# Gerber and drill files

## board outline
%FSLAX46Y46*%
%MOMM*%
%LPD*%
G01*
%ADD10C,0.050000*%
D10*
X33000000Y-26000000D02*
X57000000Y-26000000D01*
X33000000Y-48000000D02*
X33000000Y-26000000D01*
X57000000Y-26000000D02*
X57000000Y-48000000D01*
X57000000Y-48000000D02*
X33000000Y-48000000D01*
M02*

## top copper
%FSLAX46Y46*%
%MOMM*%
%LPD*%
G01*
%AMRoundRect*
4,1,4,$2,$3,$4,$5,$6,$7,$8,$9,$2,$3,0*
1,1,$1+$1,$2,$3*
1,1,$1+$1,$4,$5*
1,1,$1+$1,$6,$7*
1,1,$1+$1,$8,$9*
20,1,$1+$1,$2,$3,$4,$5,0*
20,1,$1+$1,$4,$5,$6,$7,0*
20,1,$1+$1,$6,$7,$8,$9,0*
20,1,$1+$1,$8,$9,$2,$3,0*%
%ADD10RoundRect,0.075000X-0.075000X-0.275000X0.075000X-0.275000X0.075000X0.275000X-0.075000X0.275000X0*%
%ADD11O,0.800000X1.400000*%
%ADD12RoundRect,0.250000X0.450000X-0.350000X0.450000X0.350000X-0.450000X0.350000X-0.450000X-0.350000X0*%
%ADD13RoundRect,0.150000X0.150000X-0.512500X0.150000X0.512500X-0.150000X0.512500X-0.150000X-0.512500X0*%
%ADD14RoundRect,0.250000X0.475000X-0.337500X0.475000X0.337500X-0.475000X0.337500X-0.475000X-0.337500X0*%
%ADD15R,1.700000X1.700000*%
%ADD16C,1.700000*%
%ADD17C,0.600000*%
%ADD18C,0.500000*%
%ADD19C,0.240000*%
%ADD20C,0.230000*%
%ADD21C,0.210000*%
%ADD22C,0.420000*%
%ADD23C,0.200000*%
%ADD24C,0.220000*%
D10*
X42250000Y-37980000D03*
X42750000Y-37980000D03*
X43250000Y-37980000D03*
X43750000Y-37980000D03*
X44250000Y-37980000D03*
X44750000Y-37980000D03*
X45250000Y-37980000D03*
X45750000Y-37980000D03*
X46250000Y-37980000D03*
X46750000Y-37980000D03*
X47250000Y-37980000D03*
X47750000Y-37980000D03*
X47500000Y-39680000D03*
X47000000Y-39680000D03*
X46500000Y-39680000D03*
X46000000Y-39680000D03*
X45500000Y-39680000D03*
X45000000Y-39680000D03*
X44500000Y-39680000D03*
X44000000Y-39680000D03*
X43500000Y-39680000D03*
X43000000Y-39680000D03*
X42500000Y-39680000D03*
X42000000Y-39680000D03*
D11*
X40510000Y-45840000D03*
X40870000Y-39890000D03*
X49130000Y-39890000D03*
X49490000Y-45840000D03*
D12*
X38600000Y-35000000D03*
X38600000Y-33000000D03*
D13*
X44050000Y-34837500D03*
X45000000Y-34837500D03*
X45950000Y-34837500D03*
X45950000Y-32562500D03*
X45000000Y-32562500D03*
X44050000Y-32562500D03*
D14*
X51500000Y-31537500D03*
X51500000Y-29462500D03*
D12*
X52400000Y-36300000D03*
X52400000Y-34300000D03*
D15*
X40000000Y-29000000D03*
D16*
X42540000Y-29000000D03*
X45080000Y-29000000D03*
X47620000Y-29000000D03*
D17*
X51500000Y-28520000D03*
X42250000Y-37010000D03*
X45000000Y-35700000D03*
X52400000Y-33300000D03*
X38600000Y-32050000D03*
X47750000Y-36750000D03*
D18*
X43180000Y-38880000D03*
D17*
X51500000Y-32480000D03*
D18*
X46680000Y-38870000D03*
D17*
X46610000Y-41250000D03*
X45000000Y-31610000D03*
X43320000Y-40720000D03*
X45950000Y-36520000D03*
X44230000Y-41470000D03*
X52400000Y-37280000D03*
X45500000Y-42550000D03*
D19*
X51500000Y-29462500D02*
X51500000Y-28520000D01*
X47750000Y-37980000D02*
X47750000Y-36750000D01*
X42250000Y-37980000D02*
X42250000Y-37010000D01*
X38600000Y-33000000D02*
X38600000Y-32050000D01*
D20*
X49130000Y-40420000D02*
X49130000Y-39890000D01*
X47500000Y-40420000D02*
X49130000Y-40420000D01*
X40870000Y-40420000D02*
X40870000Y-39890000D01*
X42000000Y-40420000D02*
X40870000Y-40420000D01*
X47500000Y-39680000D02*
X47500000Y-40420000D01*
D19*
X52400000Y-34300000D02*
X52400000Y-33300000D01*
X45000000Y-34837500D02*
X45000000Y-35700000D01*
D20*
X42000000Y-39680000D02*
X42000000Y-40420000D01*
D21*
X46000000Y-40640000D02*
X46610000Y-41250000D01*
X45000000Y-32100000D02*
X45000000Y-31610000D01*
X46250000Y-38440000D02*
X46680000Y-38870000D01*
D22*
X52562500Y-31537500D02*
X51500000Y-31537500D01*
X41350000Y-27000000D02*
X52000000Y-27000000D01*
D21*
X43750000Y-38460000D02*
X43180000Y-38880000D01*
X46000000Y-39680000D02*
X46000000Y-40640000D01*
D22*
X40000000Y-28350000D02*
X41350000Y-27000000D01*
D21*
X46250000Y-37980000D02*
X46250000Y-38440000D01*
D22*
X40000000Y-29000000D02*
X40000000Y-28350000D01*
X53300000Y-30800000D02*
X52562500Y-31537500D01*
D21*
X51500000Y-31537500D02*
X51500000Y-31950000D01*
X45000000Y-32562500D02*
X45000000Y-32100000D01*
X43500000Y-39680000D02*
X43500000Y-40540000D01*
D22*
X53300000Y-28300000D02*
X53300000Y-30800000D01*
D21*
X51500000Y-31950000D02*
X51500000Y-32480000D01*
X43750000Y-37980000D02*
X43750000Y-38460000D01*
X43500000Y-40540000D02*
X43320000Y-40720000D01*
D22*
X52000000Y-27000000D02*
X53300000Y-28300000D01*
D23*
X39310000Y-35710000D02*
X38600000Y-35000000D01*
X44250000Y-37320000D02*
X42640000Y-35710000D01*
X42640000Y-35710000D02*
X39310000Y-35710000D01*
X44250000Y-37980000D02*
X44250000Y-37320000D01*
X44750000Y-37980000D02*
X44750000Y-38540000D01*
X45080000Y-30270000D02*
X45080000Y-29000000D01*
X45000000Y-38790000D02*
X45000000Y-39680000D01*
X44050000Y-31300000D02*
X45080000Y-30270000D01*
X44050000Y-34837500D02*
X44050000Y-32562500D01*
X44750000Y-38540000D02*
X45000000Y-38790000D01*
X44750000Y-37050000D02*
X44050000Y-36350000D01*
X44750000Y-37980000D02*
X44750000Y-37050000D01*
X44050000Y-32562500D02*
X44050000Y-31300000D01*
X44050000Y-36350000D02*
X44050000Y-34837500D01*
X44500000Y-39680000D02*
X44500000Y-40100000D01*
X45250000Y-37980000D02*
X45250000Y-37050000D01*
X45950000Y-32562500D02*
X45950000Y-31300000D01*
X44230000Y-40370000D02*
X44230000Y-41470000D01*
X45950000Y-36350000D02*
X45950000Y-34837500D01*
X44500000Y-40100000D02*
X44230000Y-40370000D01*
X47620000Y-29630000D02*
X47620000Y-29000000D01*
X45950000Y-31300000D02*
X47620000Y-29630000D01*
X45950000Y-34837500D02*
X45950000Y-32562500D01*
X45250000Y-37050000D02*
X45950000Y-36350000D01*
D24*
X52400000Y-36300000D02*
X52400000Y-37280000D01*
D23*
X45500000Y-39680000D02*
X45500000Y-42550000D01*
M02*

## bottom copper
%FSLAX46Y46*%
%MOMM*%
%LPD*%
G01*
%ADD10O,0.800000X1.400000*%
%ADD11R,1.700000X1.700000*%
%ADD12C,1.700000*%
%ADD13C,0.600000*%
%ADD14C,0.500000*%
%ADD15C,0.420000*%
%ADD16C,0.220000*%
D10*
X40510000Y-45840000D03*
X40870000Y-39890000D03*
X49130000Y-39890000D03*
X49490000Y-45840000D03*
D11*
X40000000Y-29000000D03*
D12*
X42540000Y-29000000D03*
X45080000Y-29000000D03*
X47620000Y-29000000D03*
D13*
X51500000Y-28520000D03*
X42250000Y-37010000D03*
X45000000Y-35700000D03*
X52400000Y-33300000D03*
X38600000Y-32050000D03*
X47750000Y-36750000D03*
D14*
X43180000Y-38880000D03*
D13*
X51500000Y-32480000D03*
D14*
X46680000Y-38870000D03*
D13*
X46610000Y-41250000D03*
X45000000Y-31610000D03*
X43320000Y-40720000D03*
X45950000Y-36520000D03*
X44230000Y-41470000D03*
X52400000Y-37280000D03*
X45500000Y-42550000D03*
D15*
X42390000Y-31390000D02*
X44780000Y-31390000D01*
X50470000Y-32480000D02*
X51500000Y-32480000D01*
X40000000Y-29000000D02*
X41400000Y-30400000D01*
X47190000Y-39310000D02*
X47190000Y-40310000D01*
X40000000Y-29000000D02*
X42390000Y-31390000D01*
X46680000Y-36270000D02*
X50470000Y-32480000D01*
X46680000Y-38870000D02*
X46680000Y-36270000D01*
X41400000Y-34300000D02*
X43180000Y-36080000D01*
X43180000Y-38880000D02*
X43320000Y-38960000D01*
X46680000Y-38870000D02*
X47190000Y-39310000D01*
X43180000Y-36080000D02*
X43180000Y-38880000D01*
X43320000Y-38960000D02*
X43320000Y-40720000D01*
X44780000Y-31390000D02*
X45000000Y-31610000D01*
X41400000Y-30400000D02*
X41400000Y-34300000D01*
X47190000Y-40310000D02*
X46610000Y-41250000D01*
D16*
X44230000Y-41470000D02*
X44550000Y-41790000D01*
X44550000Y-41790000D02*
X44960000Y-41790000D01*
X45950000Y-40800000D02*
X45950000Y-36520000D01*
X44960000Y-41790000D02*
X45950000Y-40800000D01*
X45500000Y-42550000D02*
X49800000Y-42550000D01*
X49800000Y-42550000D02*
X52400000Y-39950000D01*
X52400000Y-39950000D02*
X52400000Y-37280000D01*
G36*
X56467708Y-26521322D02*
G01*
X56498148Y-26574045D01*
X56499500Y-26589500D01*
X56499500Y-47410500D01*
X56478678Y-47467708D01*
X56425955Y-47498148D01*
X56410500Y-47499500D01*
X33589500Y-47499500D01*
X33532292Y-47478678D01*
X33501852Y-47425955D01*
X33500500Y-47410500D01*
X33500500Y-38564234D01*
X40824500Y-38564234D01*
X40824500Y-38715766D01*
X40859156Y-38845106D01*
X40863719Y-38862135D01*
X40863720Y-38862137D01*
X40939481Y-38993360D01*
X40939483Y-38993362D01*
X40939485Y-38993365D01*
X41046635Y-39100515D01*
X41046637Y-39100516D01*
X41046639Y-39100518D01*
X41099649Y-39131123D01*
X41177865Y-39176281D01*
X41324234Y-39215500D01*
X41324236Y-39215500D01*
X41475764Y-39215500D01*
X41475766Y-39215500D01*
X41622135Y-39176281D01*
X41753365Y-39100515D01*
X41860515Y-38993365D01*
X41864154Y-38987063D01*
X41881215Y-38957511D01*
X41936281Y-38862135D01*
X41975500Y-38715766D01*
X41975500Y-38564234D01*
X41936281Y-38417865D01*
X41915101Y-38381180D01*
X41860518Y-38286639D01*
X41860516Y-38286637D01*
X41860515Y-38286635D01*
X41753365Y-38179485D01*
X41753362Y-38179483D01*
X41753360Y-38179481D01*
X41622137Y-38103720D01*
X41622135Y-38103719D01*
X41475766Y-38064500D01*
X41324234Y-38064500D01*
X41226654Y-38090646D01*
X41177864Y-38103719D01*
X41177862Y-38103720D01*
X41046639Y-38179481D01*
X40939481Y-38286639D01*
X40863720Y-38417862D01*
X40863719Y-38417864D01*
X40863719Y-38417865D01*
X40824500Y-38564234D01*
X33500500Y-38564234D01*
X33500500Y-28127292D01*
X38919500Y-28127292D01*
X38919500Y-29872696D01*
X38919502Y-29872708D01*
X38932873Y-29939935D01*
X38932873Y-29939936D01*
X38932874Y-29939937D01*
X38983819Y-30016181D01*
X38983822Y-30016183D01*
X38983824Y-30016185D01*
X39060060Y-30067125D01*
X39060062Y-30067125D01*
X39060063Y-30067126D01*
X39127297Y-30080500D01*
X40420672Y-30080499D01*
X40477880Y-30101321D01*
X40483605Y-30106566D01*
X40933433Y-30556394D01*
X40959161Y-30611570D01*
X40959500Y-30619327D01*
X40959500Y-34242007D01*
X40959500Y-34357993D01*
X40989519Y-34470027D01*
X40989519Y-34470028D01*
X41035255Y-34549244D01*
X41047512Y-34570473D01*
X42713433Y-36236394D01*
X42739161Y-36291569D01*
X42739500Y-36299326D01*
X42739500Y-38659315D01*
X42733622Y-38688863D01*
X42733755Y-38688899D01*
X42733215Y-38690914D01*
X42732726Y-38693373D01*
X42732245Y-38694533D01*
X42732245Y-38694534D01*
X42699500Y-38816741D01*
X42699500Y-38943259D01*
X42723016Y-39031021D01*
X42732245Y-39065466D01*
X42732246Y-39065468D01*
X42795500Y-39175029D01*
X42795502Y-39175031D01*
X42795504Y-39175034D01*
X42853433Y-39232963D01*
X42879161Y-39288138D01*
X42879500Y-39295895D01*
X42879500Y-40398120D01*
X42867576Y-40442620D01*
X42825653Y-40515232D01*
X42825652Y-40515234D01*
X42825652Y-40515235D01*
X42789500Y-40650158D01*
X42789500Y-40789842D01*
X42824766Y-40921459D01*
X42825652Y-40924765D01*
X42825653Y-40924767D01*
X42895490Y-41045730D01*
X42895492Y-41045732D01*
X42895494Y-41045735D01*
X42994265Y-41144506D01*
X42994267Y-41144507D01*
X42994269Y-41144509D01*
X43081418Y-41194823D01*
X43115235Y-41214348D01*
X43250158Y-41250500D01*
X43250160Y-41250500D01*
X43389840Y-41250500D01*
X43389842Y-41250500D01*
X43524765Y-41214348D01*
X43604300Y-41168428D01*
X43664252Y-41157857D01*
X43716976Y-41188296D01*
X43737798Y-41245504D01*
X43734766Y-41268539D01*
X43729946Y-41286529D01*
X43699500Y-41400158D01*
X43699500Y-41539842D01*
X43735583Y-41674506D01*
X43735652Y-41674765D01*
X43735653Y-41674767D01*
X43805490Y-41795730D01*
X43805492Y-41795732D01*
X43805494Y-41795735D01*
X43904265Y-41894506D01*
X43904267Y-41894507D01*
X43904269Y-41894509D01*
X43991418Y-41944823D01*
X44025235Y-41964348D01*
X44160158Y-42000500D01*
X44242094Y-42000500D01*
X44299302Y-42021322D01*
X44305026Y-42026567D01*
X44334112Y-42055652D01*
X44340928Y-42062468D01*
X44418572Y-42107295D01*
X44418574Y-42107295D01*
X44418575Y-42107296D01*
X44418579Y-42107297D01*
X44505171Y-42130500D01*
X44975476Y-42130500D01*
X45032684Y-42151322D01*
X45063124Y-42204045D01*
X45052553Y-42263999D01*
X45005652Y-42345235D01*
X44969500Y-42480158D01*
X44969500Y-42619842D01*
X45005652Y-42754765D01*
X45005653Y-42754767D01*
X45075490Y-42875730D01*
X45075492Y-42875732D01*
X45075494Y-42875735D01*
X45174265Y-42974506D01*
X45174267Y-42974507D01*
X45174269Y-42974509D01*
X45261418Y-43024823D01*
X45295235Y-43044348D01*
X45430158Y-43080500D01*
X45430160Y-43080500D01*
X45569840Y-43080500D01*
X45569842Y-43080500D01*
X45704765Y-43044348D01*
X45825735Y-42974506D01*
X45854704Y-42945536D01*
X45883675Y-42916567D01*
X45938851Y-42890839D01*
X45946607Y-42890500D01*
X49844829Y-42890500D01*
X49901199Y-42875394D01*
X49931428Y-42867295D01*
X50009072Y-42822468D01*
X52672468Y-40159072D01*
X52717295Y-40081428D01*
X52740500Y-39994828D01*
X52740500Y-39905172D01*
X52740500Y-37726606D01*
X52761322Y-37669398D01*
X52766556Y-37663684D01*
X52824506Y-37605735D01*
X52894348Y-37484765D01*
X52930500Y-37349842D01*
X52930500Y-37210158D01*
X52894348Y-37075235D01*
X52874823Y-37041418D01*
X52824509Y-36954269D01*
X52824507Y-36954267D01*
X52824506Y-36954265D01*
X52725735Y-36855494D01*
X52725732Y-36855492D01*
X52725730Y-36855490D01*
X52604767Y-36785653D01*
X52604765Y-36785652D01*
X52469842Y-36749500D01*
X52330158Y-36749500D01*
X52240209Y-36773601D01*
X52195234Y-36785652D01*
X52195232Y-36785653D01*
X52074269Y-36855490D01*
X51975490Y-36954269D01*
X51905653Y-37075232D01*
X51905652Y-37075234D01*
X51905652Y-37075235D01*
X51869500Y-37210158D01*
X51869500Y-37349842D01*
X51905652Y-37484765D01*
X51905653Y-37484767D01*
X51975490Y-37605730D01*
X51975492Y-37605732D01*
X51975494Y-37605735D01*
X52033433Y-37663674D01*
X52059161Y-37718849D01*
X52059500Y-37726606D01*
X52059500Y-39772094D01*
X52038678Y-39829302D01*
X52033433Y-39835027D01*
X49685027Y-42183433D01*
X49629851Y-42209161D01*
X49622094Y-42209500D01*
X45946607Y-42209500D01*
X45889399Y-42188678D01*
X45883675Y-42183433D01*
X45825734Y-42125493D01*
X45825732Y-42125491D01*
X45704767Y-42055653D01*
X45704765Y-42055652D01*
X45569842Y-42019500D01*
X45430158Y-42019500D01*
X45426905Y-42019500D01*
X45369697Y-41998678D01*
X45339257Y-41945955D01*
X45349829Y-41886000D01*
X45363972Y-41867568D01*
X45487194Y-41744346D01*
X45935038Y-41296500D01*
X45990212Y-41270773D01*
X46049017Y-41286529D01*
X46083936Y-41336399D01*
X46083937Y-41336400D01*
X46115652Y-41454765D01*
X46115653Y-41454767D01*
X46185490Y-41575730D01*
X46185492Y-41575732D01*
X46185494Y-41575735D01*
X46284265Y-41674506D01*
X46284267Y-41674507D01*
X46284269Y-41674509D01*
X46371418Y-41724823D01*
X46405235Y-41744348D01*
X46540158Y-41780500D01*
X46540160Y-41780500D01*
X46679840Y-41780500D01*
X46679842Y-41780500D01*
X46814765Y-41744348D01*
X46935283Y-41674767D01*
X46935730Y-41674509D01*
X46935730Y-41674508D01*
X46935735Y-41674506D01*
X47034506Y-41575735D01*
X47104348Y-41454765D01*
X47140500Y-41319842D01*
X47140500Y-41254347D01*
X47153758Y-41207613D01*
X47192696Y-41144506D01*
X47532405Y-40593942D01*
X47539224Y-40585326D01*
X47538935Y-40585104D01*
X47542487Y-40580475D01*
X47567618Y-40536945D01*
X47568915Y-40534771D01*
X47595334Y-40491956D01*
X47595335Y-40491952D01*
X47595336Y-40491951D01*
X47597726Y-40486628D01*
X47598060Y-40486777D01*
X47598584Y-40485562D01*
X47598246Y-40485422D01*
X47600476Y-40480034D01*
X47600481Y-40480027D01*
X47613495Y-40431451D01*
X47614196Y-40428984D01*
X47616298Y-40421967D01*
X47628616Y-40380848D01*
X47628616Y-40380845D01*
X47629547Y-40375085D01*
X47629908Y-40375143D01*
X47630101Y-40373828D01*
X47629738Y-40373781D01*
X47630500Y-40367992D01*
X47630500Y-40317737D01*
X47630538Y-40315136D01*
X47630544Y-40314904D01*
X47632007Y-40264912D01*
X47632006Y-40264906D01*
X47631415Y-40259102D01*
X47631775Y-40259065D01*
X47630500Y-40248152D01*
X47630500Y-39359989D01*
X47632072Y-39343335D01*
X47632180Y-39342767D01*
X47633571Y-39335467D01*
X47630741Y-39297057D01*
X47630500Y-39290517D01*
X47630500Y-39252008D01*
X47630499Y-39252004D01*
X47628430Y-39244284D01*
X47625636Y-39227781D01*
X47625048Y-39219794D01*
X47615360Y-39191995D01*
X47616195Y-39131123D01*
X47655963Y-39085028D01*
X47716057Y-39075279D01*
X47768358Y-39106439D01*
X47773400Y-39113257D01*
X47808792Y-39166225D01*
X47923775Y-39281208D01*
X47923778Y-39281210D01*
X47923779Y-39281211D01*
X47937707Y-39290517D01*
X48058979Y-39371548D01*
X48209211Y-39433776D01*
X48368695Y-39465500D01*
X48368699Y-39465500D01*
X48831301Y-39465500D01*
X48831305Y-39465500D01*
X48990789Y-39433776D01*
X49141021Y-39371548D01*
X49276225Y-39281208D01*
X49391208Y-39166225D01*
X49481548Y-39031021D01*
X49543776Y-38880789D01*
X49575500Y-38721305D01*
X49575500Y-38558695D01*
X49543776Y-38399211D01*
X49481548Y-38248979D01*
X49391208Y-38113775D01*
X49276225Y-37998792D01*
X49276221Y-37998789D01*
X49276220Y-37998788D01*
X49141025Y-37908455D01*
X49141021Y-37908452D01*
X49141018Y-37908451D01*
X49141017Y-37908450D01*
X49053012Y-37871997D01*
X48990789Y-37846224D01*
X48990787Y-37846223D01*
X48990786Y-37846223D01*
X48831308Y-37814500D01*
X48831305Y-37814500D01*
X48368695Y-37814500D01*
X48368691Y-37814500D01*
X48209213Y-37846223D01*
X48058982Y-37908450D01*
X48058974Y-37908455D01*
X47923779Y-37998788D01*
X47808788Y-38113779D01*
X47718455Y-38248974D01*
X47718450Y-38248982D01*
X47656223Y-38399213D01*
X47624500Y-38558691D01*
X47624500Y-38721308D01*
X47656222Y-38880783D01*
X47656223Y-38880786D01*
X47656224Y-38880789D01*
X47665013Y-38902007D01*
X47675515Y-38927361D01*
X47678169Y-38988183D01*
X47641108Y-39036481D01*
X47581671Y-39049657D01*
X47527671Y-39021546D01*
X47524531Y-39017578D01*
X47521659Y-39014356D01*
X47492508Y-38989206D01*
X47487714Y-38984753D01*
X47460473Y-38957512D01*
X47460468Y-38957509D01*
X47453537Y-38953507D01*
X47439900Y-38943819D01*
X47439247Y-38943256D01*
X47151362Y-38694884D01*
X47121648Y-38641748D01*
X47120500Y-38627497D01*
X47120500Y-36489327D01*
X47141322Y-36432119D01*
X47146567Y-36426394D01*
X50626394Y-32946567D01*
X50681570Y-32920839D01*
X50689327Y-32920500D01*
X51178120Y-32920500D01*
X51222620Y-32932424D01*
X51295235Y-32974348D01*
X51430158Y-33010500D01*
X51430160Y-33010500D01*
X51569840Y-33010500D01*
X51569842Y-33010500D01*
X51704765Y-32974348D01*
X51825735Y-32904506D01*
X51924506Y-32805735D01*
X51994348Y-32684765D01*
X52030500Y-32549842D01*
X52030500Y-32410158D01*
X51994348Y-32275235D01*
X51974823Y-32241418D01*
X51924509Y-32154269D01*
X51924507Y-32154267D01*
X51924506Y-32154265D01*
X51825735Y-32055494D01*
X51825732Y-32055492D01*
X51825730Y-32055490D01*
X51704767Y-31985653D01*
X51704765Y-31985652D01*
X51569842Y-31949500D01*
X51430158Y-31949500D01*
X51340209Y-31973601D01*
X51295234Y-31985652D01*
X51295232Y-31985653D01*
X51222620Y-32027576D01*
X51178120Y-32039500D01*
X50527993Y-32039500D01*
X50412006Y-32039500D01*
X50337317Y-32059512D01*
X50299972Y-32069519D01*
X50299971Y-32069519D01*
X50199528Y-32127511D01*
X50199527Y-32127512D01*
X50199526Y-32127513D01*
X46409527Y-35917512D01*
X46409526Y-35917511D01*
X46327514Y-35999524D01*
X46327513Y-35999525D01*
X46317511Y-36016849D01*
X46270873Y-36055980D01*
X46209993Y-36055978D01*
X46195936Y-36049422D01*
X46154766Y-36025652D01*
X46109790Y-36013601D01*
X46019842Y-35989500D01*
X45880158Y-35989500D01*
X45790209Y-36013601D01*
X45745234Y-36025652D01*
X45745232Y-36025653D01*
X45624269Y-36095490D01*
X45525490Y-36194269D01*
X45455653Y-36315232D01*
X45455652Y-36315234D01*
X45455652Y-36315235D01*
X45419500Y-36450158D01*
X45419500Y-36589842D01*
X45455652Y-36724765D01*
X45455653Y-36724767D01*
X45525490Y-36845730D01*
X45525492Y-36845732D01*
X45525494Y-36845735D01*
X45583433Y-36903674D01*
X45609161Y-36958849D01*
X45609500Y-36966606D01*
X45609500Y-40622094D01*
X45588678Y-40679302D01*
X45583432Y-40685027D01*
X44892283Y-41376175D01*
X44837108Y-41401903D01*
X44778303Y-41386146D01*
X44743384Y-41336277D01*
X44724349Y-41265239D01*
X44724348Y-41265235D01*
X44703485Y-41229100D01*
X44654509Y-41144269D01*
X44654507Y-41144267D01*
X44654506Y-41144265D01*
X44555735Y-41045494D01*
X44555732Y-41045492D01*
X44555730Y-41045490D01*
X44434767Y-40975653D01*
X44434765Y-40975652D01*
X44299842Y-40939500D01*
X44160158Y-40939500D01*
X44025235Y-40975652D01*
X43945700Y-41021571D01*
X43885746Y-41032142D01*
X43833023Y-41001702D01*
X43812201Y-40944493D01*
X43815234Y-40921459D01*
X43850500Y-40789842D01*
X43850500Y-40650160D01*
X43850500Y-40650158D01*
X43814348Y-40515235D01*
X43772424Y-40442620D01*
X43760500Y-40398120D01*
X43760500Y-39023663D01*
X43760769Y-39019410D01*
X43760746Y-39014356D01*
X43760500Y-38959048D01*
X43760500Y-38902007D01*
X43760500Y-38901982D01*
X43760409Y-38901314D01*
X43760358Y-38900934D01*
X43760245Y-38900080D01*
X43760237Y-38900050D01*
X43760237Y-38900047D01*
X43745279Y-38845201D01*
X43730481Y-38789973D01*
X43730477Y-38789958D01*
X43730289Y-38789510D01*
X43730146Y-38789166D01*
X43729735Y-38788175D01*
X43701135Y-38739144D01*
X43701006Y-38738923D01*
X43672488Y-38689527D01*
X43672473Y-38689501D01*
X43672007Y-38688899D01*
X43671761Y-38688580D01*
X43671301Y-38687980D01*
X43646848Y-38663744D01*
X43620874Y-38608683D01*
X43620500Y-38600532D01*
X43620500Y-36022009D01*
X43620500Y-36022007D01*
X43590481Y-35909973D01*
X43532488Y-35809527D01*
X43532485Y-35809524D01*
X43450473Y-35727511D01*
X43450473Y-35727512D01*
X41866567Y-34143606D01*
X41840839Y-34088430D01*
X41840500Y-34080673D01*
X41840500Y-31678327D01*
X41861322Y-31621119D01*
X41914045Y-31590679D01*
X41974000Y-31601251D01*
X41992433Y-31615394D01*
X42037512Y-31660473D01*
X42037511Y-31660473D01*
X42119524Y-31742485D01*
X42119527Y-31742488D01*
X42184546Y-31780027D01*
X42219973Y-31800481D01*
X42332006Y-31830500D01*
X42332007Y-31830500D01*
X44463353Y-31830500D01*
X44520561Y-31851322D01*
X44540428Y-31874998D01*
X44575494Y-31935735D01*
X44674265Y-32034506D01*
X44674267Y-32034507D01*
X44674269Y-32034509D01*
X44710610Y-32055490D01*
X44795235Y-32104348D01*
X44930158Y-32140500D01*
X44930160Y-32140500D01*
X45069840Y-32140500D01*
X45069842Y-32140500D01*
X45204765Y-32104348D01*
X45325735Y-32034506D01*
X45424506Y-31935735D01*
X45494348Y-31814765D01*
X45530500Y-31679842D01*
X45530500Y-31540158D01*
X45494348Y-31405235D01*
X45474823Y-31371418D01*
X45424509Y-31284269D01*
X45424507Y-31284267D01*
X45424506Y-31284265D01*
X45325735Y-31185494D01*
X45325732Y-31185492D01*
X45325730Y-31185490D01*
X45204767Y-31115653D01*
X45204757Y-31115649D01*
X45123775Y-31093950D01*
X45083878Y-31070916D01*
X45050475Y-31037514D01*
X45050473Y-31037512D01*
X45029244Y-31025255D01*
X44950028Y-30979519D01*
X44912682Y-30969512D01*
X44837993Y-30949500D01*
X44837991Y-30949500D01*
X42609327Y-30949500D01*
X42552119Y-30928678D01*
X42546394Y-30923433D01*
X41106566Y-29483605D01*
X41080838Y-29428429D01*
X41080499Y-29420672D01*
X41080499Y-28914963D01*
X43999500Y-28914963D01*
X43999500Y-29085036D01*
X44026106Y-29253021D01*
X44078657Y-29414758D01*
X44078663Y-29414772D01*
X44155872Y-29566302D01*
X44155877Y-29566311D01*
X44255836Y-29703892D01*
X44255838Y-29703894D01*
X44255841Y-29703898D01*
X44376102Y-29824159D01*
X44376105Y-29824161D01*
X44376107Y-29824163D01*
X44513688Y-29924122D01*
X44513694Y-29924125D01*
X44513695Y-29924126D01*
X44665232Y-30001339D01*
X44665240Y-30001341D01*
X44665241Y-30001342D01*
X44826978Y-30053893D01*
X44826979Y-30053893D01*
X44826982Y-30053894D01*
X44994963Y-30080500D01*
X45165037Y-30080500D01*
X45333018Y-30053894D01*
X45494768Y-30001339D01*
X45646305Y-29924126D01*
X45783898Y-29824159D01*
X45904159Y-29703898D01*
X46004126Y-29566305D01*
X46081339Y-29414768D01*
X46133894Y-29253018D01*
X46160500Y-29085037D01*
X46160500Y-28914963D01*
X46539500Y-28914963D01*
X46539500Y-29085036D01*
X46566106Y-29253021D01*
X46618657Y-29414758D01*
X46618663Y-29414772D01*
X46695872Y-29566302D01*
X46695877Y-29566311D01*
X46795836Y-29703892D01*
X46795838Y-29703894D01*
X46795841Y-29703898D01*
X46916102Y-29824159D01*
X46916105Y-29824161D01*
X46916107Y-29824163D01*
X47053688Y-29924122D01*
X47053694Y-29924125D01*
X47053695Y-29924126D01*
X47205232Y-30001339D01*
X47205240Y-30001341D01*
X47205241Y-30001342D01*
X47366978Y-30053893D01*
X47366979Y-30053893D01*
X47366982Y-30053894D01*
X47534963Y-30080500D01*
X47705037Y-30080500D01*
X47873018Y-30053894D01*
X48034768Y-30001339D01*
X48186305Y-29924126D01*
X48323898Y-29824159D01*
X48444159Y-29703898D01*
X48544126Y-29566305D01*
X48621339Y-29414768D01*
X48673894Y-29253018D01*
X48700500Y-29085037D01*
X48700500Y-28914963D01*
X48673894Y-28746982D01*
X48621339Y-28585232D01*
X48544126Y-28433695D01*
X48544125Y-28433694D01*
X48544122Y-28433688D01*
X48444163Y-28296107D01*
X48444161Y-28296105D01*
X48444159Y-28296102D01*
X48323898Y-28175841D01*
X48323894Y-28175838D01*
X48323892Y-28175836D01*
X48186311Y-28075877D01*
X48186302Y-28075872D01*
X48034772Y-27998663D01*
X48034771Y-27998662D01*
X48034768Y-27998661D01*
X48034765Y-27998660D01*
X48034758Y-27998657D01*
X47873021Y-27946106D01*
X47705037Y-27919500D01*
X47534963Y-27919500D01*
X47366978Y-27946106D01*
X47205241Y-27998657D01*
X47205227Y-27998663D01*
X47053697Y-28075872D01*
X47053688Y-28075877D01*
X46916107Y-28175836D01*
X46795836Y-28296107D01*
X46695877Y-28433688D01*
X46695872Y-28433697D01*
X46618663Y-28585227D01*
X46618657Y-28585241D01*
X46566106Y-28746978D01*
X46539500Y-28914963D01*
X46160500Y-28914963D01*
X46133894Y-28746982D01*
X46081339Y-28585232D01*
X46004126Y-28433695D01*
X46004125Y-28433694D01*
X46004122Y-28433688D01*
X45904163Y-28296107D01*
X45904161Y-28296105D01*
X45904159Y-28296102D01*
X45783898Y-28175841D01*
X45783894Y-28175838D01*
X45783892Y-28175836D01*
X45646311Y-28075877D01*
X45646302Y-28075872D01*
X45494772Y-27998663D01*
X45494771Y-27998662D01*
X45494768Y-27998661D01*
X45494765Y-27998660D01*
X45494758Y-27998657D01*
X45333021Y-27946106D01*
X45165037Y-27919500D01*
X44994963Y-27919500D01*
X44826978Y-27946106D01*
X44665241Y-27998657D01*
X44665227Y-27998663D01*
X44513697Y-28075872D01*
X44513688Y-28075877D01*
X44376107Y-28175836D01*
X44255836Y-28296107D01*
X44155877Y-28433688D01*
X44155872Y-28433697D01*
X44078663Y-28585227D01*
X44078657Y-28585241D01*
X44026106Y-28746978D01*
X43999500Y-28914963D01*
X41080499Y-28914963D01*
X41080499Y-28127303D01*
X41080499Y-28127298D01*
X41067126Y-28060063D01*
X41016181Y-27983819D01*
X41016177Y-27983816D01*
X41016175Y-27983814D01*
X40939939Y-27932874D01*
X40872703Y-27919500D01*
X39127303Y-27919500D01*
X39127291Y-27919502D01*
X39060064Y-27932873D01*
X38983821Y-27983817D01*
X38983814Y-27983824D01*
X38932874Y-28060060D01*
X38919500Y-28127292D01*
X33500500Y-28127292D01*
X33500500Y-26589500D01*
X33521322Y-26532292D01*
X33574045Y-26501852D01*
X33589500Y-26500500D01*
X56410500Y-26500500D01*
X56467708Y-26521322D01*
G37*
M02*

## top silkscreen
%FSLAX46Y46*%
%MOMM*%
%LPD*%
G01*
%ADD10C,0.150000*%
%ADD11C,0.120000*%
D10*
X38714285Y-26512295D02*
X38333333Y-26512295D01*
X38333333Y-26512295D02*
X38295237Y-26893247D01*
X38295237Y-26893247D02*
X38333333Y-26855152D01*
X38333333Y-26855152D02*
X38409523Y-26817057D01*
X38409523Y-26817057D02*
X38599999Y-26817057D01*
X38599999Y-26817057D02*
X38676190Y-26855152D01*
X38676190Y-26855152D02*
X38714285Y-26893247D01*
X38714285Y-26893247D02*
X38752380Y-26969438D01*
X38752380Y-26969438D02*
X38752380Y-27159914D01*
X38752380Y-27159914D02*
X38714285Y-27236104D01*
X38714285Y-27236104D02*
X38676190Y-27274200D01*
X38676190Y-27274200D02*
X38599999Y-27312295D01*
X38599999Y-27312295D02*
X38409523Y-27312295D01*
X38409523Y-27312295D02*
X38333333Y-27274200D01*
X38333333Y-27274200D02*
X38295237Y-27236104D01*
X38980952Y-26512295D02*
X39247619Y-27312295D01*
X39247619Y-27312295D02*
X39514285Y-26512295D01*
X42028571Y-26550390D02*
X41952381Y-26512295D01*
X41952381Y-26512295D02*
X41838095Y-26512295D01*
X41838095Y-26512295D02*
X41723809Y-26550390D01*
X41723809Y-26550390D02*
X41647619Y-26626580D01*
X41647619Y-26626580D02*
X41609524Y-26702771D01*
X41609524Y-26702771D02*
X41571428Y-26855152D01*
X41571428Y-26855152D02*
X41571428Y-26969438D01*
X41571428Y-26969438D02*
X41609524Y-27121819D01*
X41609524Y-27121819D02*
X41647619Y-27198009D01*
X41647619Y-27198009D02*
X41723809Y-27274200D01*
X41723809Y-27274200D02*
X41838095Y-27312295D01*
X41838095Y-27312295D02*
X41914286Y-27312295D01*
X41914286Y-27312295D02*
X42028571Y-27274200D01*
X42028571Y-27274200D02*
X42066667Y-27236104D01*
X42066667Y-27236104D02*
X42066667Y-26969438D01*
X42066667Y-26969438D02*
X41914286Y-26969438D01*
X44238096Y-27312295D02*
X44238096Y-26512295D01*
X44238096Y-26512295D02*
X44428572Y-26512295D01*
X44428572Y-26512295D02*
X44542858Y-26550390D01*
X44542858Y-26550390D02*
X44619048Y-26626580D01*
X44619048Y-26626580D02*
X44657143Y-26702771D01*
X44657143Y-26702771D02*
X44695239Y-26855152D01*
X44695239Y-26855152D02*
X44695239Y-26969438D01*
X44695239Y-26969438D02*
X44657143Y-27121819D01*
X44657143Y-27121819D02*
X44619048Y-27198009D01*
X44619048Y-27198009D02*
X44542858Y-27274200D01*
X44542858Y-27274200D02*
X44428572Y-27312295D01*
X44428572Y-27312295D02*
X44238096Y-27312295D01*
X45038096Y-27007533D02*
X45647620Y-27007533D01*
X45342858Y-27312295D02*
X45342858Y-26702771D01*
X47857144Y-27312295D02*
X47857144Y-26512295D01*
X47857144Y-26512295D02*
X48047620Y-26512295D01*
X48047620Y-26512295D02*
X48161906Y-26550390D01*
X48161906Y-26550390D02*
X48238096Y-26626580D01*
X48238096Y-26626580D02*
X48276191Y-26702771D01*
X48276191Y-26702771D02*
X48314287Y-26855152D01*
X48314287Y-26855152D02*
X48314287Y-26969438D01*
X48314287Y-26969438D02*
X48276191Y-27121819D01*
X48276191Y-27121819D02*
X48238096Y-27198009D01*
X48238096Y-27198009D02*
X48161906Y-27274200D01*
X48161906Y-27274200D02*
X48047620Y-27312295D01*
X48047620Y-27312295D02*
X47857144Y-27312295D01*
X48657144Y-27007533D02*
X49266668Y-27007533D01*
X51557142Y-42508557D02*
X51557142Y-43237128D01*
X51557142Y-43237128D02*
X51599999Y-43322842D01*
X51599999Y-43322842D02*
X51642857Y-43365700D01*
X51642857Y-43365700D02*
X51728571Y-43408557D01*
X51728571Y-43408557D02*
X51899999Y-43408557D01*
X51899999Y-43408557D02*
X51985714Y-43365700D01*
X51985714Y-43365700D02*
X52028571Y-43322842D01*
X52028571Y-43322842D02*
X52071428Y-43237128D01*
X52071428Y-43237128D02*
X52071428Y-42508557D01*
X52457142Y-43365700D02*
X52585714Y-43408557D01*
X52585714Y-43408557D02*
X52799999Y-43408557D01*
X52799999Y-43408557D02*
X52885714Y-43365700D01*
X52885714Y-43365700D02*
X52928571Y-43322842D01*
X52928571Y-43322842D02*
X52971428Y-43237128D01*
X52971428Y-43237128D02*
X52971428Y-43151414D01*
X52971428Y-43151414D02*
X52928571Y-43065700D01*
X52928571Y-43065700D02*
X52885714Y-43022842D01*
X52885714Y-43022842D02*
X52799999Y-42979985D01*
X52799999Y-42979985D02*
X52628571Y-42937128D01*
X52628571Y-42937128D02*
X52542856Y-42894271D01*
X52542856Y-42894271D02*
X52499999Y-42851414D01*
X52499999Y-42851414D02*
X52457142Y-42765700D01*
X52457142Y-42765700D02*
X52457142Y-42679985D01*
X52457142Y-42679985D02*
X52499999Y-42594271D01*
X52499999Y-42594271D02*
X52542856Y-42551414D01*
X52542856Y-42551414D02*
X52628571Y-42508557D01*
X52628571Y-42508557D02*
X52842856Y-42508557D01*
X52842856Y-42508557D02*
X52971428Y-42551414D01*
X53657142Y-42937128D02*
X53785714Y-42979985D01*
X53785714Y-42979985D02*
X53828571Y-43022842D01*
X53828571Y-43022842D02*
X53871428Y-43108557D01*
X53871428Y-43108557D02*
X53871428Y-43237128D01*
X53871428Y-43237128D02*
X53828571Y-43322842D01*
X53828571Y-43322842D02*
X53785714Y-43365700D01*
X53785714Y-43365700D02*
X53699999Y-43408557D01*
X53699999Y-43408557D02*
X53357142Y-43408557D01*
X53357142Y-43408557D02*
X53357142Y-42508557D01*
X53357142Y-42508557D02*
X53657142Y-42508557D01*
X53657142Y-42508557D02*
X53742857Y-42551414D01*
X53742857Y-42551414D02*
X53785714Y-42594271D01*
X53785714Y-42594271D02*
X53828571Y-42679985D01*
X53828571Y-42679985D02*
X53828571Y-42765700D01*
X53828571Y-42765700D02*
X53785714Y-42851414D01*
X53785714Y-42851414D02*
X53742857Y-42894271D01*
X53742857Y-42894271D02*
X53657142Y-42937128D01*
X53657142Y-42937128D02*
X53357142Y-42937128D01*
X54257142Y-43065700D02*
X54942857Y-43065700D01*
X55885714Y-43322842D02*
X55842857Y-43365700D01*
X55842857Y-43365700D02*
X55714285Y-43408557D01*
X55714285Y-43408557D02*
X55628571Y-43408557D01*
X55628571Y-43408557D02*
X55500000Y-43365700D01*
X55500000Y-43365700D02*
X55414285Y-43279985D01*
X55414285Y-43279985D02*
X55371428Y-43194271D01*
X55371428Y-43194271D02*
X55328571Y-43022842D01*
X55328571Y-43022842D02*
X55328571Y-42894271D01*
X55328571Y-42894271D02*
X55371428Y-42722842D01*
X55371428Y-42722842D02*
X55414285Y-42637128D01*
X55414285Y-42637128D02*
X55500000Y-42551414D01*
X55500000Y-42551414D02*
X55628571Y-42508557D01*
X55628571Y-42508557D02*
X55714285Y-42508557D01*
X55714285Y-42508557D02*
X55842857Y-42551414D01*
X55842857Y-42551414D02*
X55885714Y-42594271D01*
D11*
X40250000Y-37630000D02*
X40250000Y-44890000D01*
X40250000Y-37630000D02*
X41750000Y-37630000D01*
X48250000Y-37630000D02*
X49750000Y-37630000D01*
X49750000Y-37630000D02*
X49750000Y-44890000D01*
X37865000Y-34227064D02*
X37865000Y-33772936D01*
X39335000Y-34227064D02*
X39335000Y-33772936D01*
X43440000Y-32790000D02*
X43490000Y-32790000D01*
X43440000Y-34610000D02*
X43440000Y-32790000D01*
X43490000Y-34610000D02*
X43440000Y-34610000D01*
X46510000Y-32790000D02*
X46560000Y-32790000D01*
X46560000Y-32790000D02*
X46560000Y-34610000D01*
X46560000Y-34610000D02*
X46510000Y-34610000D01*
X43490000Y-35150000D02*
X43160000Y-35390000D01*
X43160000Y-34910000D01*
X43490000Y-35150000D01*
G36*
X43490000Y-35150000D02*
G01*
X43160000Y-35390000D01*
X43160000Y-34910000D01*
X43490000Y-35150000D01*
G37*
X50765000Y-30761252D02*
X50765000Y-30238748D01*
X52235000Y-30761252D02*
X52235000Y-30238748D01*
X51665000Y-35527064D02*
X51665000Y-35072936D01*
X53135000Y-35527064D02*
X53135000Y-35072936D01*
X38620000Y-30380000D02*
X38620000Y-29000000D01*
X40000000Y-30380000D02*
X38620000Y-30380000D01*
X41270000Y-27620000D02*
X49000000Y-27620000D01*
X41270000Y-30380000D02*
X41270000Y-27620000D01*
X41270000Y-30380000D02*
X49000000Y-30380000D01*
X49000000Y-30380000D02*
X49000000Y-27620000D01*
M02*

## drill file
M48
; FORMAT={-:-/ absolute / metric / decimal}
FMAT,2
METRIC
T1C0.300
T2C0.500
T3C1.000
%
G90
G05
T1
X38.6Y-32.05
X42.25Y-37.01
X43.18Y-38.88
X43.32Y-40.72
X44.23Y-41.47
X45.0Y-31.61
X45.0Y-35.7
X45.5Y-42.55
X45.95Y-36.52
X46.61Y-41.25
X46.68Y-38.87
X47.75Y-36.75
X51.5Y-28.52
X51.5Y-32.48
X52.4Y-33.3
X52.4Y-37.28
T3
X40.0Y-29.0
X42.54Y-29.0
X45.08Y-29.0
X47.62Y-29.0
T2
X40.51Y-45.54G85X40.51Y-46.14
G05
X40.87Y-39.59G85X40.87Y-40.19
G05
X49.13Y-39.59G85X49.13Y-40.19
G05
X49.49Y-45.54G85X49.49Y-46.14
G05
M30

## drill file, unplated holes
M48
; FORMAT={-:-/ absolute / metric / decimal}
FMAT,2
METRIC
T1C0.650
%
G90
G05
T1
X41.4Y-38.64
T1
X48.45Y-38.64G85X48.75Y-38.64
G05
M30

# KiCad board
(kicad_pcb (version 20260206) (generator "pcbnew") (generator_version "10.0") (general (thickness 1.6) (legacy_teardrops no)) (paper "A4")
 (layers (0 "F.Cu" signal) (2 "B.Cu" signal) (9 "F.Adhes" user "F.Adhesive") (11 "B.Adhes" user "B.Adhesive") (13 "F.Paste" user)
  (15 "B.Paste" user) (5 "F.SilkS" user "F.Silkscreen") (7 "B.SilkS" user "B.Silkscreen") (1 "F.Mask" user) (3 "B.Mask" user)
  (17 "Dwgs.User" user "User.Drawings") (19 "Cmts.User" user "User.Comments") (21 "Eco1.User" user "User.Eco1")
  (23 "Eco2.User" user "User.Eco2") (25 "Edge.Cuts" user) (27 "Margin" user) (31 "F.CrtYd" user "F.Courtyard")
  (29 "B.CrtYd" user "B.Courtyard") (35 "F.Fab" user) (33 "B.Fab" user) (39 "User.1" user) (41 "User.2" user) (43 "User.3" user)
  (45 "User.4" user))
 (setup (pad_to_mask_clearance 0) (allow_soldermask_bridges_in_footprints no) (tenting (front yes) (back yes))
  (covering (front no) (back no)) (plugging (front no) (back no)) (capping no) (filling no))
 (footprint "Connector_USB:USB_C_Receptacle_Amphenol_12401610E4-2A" (layer "F.Cu") (at 45 43)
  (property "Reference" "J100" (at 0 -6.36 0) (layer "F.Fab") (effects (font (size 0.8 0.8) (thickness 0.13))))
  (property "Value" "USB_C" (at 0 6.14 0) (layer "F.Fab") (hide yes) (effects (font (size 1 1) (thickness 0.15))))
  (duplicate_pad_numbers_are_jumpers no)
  (fp_line (start -4.75 -5.37) (end -4.75 1.89) (stroke (width 0.12) (type solid)) (layer "F.SilkS"))
  (fp_line (start -4.75 -5.37) (end -3.25 -5.37) (stroke (width 0.12) (type solid)) (layer "F.SilkS"))
  (fp_line (start 3.25 -5.37) (end 4.75 -5.37) (stroke (width 0.12) (type solid)) (layer "F.SilkS"))
  (fp_line (start 4.75 -5.37) (end 4.75 1.89) (stroke (width 0.12) (type solid)) (layer "F.SilkS"))
  (pad "" np_thru_hole circle (at -3.6 -4.36) (size 0.65 0.65) (drill 0.65) (layers "*.Cu" "*.Mask"))
  (pad "" np_thru_hole oval (at 3.6 -4.36) (size 0.95 0.65) (drill oval 0.95 0.65) (layers "*.Cu" "*.Mask"))
  (pad "A1" smd roundrect (at -2.75 -5.02) (size 0.3 0.7) (layers "F.Cu" "F.Mask" "F.Paste") (roundrect_rratio 0.25) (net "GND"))
  (pad "A2" smd roundrect (at -2.25 -5.02) (size 0.3 0.7) (layers "F.Cu" "F.Mask" "F.Paste") (roundrect_rratio 0.25))
  (pad "A3" smd roundrect (at -1.75 -5.02) (size 0.3 0.7) (layers "F.Cu" "F.Mask" "F.Paste") (roundrect_rratio 0.25))
  (pad "A4" smd roundrect (at -1.25 -5.02) (size 0.3 0.7) (layers "F.Cu" "F.Mask" "F.Paste") (roundrect_rratio 0.25) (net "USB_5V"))
  (pad "A5" smd roundrect (at -0.75 -5.02) (size 0.3 0.7) (layers "F.Cu" "F.Mask" "F.Paste") (roundrect_rratio 0.25) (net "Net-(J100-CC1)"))
  (pad "A6" smd roundrect (at -0.25 -5.02) (size 0.3 0.7) (layers "F.Cu" "F.Mask" "F.Paste") (roundrect_rratio 0.25) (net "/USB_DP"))
  (pad "A7" smd roundrect (at 0.25 -5.02) (size 0.3 0.7) (layers "F.Cu" "F.Mask" "F.Paste") (roundrect_rratio 0.25) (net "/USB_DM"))
  (pad "A8" smd roundrect (at 0.75 -5.02) (size 0.3 0.7) (layers "F.Cu" "F.Mask" "F.Paste") (roundrect_rratio 0.25))
  (pad "A9" smd roundrect (at 1.25 -5.02) (size 0.3 0.7) (layers "F.Cu" "F.Mask" "F.Paste") (roundrect_rratio 0.25) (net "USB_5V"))
  (pad "A10" smd roundrect (at 1.75 -5.02) (size 0.3 0.7) (layers "F.Cu" "F.Mask" "F.Paste") (roundrect_rratio 0.25))
  (pad "A11" smd roundrect (at 2.25 -5.02) (size 0.3 0.7) (layers "F.Cu" "F.Mask" "F.Paste") (roundrect_rratio 0.25))
  (pad "A12" smd roundrect (at 2.75 -5.02) (size 0.3 0.7) (layers "F.Cu" "F.Mask" "F.Paste") (roundrect_rratio 0.25) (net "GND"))
  (pad "B1" smd roundrect (at 2.5 -3.32) (size 0.3 0.7) (layers "F.Cu" "F.Mask" "F.Paste") (roundrect_rratio 0.25) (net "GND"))
  (pad "B2" smd roundrect (at 2 -3.32) (size 0.3 0.7) (layers "F.Cu" "F.Mask" "F.Paste") (roundrect_rratio 0.25))
  (pad "B3" smd roundrect (at 1.5 -3.32) (size 0.3 0.7) (layers "F.Cu" "F.Mask" "F.Paste") (roundrect_rratio 0.25))
  (pad "B4" smd roundrect (at 1 -3.32) (size 0.3 0.7) (layers "F.Cu" "F.Mask" "F.Paste") (roundrect_rratio 0.25) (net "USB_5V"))
  (pad "B5" smd roundrect (at 0.5 -3.32) (size 0.3 0.7) (layers "F.Cu" "F.Mask" "F.Paste") (roundrect_rratio 0.25) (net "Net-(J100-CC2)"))
  (pad "B6" smd roundrect (at 0 -3.32) (size 0.3 0.7) (layers "F.Cu" "F.Mask" "F.Paste") (roundrect_rratio 0.25) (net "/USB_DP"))
  (pad "B7" smd roundrect (at -0.5 -3.32) (size 0.3 0.7) (layers "F.Cu" "F.Mask" "F.Paste") (roundrect_rratio 0.25) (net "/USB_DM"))
  (pad "B8" smd roundrect (at -1 -3.32) (size 0.3 0.7) (layers "F.Cu" "F.Mask" "F.Paste") (roundrect_rratio 0.25))
  (pad "B9" smd roundrect (at -1.5 -3.32) (size 0.3 0.7) (layers "F.Cu" "F.Mask" "F.Paste") (roundrect_rratio 0.25) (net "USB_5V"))
  (pad "B10" smd roundrect (at -2 -3.32) (size 0.3 0.7) (layers "F.Cu" "F.Mask" "F.Paste") (roundrect_rratio 0.25))
  (pad "B11" smd roundrect (at -2.5 -3.32) (size 0.3 0.7) (layers "F.Cu" "F.Mask" "F.Paste") (roundrect_rratio 0.25))
  (pad "B12" smd roundrect (at -3 -3.32) (size 0.3 0.7) (layers "F.Cu" "F.Mask" "F.Paste") (roundrect_rratio 0.25) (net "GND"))
  (pad "SH" thru_hole oval (at -4.49 2.84) (size 0.8 1.4) (drill oval 0.5 1.1) (layers "*.Cu" "*.Mask") (remove_unused_layers no)
   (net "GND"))
  (pad "SH" thru_hole oval (at -4.13 -3.11) (size 0.8 1.4) (drill oval 0.5 1.1) (layers "*.Cu" "*.Mask") (remove_unused_layers no)
   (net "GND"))
  (pad "SH" thru_hole oval (at 4.13 -3.11) (size 0.8 1.4) (drill oval 0.5 1.1) (layers "*.Cu" "*.Mask") (remove_unused_layers no)
   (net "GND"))
  (pad "SH" thru_hole oval (at 4.49 2.84) (size 0.8 1.4) (drill oval 0.5 1.1) (layers "*.Cu" "*.Mask") (remove_unused_layers no) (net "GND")))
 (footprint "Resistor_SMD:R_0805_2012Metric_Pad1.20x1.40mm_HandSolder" (layer "F.Cu") (at 38.6 34 90)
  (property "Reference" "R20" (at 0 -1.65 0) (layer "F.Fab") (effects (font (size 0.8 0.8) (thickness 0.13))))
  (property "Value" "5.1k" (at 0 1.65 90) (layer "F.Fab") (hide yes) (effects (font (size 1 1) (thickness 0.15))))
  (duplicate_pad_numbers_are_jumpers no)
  (fp_line (start -0.227064 -0.735) (end 0.227064 -0.735) (stroke (width 0.12) (type solid)) (layer "F.SilkS"))
  (fp_line (start -0.227064 0.735) (end 0.227064 0.735) (stroke (width 0.12) (type solid)) (layer "F.SilkS"))
  (pad "1" smd roundrect (at -1 0 90) (size 1.2 1.4) (layers "F.Cu" "F.Mask" "F.Paste") (roundrect_rratio 0.208333) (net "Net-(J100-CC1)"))
  (pad "2" smd roundrect (at 1 0 90) (size 1.2 1.4) (layers "F.Cu" "F.Mask" "F.Paste") (roundrect_rratio 0.208333) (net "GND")))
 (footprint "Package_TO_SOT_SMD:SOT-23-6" (layer "F.Cu") (at 45 33.7 90)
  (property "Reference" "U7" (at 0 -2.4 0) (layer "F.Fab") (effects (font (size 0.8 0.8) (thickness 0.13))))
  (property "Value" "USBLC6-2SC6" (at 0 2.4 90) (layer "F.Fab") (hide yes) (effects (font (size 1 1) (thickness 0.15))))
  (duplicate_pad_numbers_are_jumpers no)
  (fp_line (start 0.91 -1.56) (end 0.91 -1.51) (stroke (width 0.12) (type solid)) (layer "F.SilkS"))
  (fp_line (start -0.91 -1.56) (end 0.91 -1.56) (stroke (width 0.12) (type solid)) (layer "F.SilkS"))
  (fp_line (start -0.91 -1.51) (end -0.91 -1.56) (stroke (width 0.12) (type solid)) (layer "F.SilkS"))
  (fp_line (start 0.91 1.51) (end 0.91 1.56) (stroke (width 0.12) (type solid)) (layer "F.SilkS"))
  (fp_line (start 0.91 1.56) (end -0.91 1.56) (stroke (width 0.12) (type solid)) (layer "F.SilkS"))
  (fp_line (start -0.91 1.56) (end -0.91 1.51) (stroke (width 0.12) (type solid)) (layer "F.SilkS"))
  (fp_poly (pts (xy -1.45 -1.51) (xy -1.69 -1.84) (xy -1.21 -1.84)) (stroke (width 0.12) (type solid)) (fill yes) (layer "F.SilkS"))
  (pad "1" smd roundrect (at -1.1375 -0.95 90) (size 1.325 0.6) (layers "F.Cu" "F.Mask" "F.Paste") (roundrect_rratio 0.25) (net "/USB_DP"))
  (pad "2" smd roundrect (at -1.1375 0 90) (size 1.325 0.6) (layers "F.Cu" "F.Mask" "F.Paste") (roundrect_rratio 0.25) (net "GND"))
  (pad "3" smd roundrect (at -1.1375 0.95 90) (size 1.325 0.6) (layers "F.Cu" "F.Mask" "F.Paste") (roundrect_rratio 0.25) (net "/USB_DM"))
  (pad "4" smd roundrect (at 1.1375 0.95 90) (size 1.325 0.6) (layers "F.Cu" "F.Mask" "F.Paste") (roundrect_rratio 0.25) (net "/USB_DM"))
  (pad "5" smd roundrect (at 1.1375 0 90) (size 1.325 0.6) (layers "F.Cu" "F.Mask" "F.Paste") (roundrect_rratio 0.25) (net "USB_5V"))
  (pad "6" smd roundrect (at 1.1375 -0.95 90) (size 1.325 0.6) (layers "F.Cu" "F.Mask" "F.Paste") (roundrect_rratio 0.25) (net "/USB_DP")))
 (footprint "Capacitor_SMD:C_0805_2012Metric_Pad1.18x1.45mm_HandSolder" (layer "F.Cu") (at 51.5 30.5 90)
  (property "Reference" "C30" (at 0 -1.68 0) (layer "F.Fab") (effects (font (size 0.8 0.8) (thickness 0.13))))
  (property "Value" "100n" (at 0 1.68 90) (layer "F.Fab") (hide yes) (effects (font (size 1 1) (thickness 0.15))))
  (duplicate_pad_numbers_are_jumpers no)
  (fp_line (start -0.261252 -0.735) (end 0.261252 -0.735) (stroke (width 0.12) (type solid)) (layer "F.SilkS"))
  (fp_line (start -0.261252 0.735) (end 0.261252 0.735) (stroke (width 0.12) (type solid)) (layer "F.SilkS"))
  (pad "1" smd roundrect (at -1.0375 0 90) (size 1.175 1.45) (layers "F.Cu" "F.Mask" "F.Paste") (roundrect_rratio 0.212766) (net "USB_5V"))
  (pad "2" smd roundrect (at 1.0375 0 90) (size 1.175 1.45) (layers "F.Cu" "F.Mask" "F.Paste") (roundrect_rratio 0.212766) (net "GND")))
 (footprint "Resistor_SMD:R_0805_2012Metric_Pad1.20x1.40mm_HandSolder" (layer "F.Cu") (at 52.4 35.3 90)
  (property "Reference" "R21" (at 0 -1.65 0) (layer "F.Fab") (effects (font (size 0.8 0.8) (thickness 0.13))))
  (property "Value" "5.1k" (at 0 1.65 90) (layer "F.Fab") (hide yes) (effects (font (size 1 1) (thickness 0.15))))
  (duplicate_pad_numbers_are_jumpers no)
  (fp_line (start -0.227064 -0.735) (end 0.227064 -0.735) (stroke (width 0.12) (type solid)) (layer "F.SilkS"))
  (fp_line (start -0.227064 0.735) (end 0.227064 0.735) (stroke (width 0.12) (type solid)) (layer "F.SilkS"))
  (pad "1" smd roundrect (at -1 0 90) (size 1.2 1.4) (layers "F.Cu" "F.Mask" "F.Paste") (roundrect_rratio 0.208333) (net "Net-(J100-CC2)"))
  (pad "2" smd roundrect (at 1 0 90) (size 1.2 1.4) (layers "F.Cu" "F.Mask" "F.Paste") (roundrect_rratio 0.208333) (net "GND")))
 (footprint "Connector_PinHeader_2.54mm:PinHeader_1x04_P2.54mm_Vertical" (layer "F.Cu") (at 40 29 90)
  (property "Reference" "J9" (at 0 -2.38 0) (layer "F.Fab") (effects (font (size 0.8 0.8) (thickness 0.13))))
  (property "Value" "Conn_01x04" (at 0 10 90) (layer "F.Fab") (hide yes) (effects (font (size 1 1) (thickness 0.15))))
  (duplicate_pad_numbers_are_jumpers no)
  (fp_line (start -1.38 -1.38) (end 0 -1.38) (stroke (width 0.12) (type solid)) (layer "F.SilkS"))
  (fp_line (start -1.38 0) (end -1.38 -1.38) (stroke (width 0.12) (type solid)) (layer "F.SilkS"))
  (fp_line (start 1.38 1.27) (end 1.38 9) (stroke (width 0.12) (type solid)) (layer "F.SilkS"))
  (fp_line (start -1.38 1.27) (end 1.38 1.27) (stroke (width 0.12) (type solid)) (layer "F.SilkS"))
  (fp_line (start -1.38 1.27) (end -1.38 9) (stroke (width 0.12) (type solid)) (layer "F.SilkS"))
  (fp_line (start -1.38 9) (end 1.38 9) (stroke (width 0.12) (type solid)) (layer "F.SilkS"))
  (pad "1" thru_hole rect (at 0 0 90) (size 1.7 1.7) (drill 1) (layers "*.Cu" "*.Mask") (remove_unused_layers no) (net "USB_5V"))
  (pad "2" thru_hole circle (at 0 2.54 90) (size 1.7 1.7) (drill 1) (layers "*.Cu" "*.Mask") (remove_unused_layers no) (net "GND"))
  (pad "3" thru_hole circle (at 0 5.08 90) (size 1.7 1.7) (drill 1) (layers "*.Cu" "*.Mask") (remove_unused_layers no) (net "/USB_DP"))
  (pad "4" thru_hole circle (at 0 7.62 90) (size 1.7 1.7) (drill 1) (layers "*.Cu" "*.Mask") (remove_unused_layers no) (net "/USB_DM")))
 (gr_line (start 33 26) (end 57 26) (stroke (width 0.05) (type default)) (layer "Edge.Cuts"))
 (gr_line (start 33 48) (end 33 26) (stroke (width 0.05) (type default)) (layer "Edge.Cuts"))
 (gr_line (start 57 26) (end 57 48) (stroke (width 0.05) (type default)) (layer "Edge.Cuts"))
 (gr_line (start 57 48) (end 33 48) (stroke (width 0.05) (type default)) (layer "Edge.Cuts"))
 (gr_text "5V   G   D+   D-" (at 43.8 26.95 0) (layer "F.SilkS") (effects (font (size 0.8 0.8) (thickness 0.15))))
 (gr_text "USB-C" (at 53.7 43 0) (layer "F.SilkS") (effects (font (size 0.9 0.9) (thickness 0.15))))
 (segment (start 51.5 29.4625) (end 51.5 28.52) (width 0.24) (layer "F.Cu") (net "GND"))
 (segment (start 47.75 37.98) (end 47.75 36.75) (width 0.24) (layer "F.Cu") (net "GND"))
 (segment (start 42.25 37.98) (end 42.25 37.01) (width 0.24) (layer "F.Cu") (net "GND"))
 (segment (start 38.6 33) (end 38.6 32.05) (width 0.24) (layer "F.Cu") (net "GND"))
 (segment (start 49.13 40.42) (end 49.13 39.89) (width 0.23) (layer "F.Cu") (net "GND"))
 (segment (start 47.5 40.42) (end 49.13 40.42) (width 0.23) (layer "F.Cu") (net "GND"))
 (segment (start 40.87 40.42) (end 40.87 39.89) (width 0.23) (layer "F.Cu") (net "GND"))
 (segment (start 42 40.42) (end 40.87 40.42) (width 0.23) (layer "F.Cu") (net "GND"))
 (segment (start 47.5 39.68) (end 47.5 40.42) (width 0.23) (layer "F.Cu") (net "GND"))
 (segment (start 52.4 34.3) (end 52.4 33.3) (width 0.24) (layer "F.Cu") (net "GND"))
 (segment (start 45 34.8375) (end 45 35.7) (width 0.24) (layer "F.Cu") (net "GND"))
 (segment (start 42 39.68) (end 42 40.42) (width 0.23) (layer "F.Cu") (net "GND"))
 (via (at 51.5 28.52) (size 0.6) (drill 0.3) (layers "F.Cu" "B.Cu") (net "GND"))
 (via (at 42.25 37.01) (size 0.6) (drill 0.3) (layers "F.Cu" "B.Cu") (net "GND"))
 (via (at 45 35.7) (size 0.6) (drill 0.3) (layers "F.Cu" "B.Cu") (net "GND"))
 (via (at 52.4 33.3) (size 0.6) (drill 0.3) (layers "F.Cu" "B.Cu") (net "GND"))
 (via (at 38.6 32.05) (size 0.6) (drill 0.3) (layers "F.Cu" "B.Cu") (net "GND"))
 (via (at 47.75 36.75) (size 0.6) (drill 0.3) (layers "F.Cu" "B.Cu") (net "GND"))
 (segment (start 46 40.64) (end 46.61 41.25) (width 0.21) (layer "F.Cu") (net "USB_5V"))
 (segment (start 45 32.1) (end 45 31.61) (width 0.21) (layer "F.Cu") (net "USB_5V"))
 (segment (start 46.25 38.44) (end 46.68 38.87) (width 0.21) (layer "F.Cu") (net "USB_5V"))
 (segment (start 52.5625 31.5375) (end 51.5 31.5375) (width 0.42) (layer "F.Cu") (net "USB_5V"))
 (segment (start 41.35 27) (end 52 27) (width 0.42) (layer "F.Cu") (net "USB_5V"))
 (segment (start 43.75 38.46) (end 43.18 38.88) (width 0.21) (layer "F.Cu") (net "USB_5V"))
 (segment (start 46 39.68) (end 46 40.64) (width 0.21) (layer "F.Cu") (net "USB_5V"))
 (segment (start 40 28.35) (end 41.35 27) (width 0.42) (layer "F.Cu") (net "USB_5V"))
 (segment (start 46.25 37.98) (end 46.25 38.44) (width 0.21) (layer "F.Cu") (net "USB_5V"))
 (segment (start 40 29) (end 40 28.35) (width 0.42) (layer "F.Cu") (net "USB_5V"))
 (segment (start 53.3 30.8) (end 52.5625 31.5375) (width 0.42) (layer "F.Cu") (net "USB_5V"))
 (segment (start 51.5 31.5375) (end 51.5 31.95) (width 0.21) (layer "F.Cu") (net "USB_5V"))
 (segment (start 45 32.5625) (end 45 32.1) (width 0.21) (layer "F.Cu") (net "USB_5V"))
 (segment (start 43.5 39.68) (end 43.5 40.54) (width 0.21) (layer "F.Cu") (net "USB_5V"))
 (segment (start 53.3 28.3) (end 53.3 30.8) (width 0.42) (layer "F.Cu") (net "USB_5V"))
 (segment (start 51.5 31.95) (end 51.5 32.48) (width 0.21) (layer "F.Cu") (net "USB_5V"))
 (segment (start 43.75 37.98) (end 43.75 38.46) (width 0.21) (layer "F.Cu") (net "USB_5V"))
 (segment (start 43.5 40.54) (end 43.32 40.72) (width 0.21) (layer "F.Cu") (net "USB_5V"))
 (segment (start 52 27) (end 53.3 28.3) (width 0.42) (layer "F.Cu") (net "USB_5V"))
 (via (at 43.18 38.88) (size 0.5) (drill 0.3) (layers "F.Cu" "B.Cu") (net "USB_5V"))
 (via (at 51.5 32.48) (size 0.6) (drill 0.3) (layers "F.Cu" "B.Cu") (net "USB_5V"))
 (via (at 46.68 38.87) (size 0.5) (drill 0.3) (layers "F.Cu" "B.Cu") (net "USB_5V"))
 (via (at 46.61 41.25) (size 0.6) (drill 0.3) (layers "F.Cu" "B.Cu") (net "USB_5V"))
 (via (at 45 31.61) (size 0.6) (drill 0.3) (layers "F.Cu" "B.Cu") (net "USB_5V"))
 (via (at 43.32 40.72) (size 0.6) (drill 0.3) (layers "F.Cu" "B.Cu") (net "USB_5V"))
 (segment (start 42.39 31.39) (end 44.78 31.39) (width 0.42) (layer "B.Cu") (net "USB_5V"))
 (segment (start 50.47 32.48) (end 51.5 32.48) (width 0.42) (layer "B.Cu") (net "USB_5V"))
 (segment (start 40 29) (end 41.4 30.4) (width 0.42) (layer "B.Cu") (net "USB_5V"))
 (segment (start 47.19 39.31) (end 47.19 40.31) (width 0.42) (layer "B.Cu") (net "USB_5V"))
 (segment (start 40 29) (end 42.39 31.39) (width 0.42) (layer "B.Cu") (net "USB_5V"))
 (segment (start 46.68 36.27) (end 50.47 32.48) (width 0.42) (layer "B.Cu") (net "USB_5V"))
 (segment (start 46.68 38.87) (end 46.68 36.27) (width 0.42) (layer "B.Cu") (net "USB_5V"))
 (segment (start 41.4 34.3) (end 43.18 36.08) (width 0.42) (layer "B.Cu") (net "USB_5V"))
 (segment (start 43.18 38.88) (end 43.32 38.96) (width 0.42) (layer "B.Cu") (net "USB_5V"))
 (segment (start 46.68 38.87) (end 47.19 39.31) (width 0.42) (layer "B.Cu") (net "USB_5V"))
 (segment (start 43.18 36.08) (end 43.18 38.88) (width 0.42) (layer "B.Cu") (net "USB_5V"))
 (segment (start 43.32 38.96) (end 43.32 40.72) (width 0.42) (layer "B.Cu") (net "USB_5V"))
 (segment (start 44.78 31.39) (end 45 31.61) (width 0.42) (layer "B.Cu") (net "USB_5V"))
 (segment (start 41.4 30.4) (end 41.4 34.3) (width 0.42) (layer "B.Cu") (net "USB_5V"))
 (segment (start 47.19 40.31) (end 46.61 41.25) (width 0.42) (layer "B.Cu") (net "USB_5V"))
 (segment (start 39.31 35.71) (end 38.6 35) (width 0.2) (layer "F.Cu") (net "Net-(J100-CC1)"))
 (segment (start 44.25 37.32) (end 42.64 35.71) (width 0.2) (layer "F.Cu") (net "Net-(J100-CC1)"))
 (segment (start 42.64 35.71) (end 39.31 35.71) (width 0.2) (layer "F.Cu") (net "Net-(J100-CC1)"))
 (segment (start 44.25 37.98) (end 44.25 37.32) (width 0.2) (layer "F.Cu") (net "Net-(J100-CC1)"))
 (segment (start 44.75 37.98) (end 44.75 38.54) (width 0.2) (layer "F.Cu") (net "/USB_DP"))
 (segment (start 45.08 30.27) (end 45.08 29) (width 0.2) (layer "F.Cu") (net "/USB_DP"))
 (segment (start 45 38.79) (end 45 39.68) (width 0.2) (layer "F.Cu") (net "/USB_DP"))
 (segment (start 44.05 31.3) (end 45.08 30.27) (width 0.2) (layer "F.Cu") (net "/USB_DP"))
 (segment (start 44.05 34.8375) (end 44.05 32.5625) (width 0.2) (layer "F.Cu") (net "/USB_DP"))
 (segment (start 44.75 38.54) (end 45 38.79) (width 0.2) (layer "F.Cu") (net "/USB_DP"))
 (segment (start 44.75 37.05) (end 44.05 36.35) (width 0.2) (layer "F.Cu") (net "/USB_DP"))
 (segment (start 44.75 37.98) (end 44.75 37.05) (width 0.2) (layer "F.Cu") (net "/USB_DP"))
 (segment (start 44.05 32.5625) (end 44.05 31.3) (width 0.2) (layer "F.Cu") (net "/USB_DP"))
 (segment (start 44.05 36.35) (end 44.05 34.8375) (width 0.2) (layer "F.Cu") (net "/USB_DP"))
 (segment (start 44.5 39.68) (end 44.5 40.1) (width 0.2) (layer "F.Cu") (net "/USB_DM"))
 (segment (start 45.25 37.98) (end 45.25 37.05) (width 0.2) (layer "F.Cu") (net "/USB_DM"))
 (segment (start 45.95 32.5625) (end 45.95 31.3) (width 0.2) (layer "F.Cu") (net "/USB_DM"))
 (segment (start 44.23 40.37) (end 44.23 41.47) (width 0.2) (layer "F.Cu") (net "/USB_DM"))
 (segment (start 45.95 36.35) (end 45.95 34.8375) (width 0.2) (layer "F.Cu") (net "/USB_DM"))
 (segment (start 44.5 40.1) (end 44.23 40.37) (width 0.2) (layer "F.Cu") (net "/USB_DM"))
 (segment (start 47.62 29.63) (end 47.62 29) (width 0.2) (layer "F.Cu") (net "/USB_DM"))
 (segment (start 45.95 31.3) (end 47.62 29.63) (width 0.2) (layer "F.Cu") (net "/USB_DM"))
 (segment (start 45.95 34.8375) (end 45.95 32.5625) (width 0.2) (layer "F.Cu") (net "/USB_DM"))
 (segment (start 45.25 37.05) (end 45.95 36.35) (width 0.2) (layer "F.Cu") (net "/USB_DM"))
 (via (at 45.95 36.52) (size 0.6) (drill 0.3) (layers "F.Cu" "B.Cu") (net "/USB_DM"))
 (via (at 44.23 41.47) (size 0.6) (drill 0.3) (layers "F.Cu" "B.Cu") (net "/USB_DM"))
 (segment (start 44.23 41.47) (end 44.55 41.79) (width 0.22) (layer "B.Cu") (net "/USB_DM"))
 (segment (start 44.55 41.79) (end 44.96 41.79) (width 0.22) (layer "B.Cu") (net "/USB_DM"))
 (segment (start 45.95 40.8) (end 45.95 36.52) (width 0.22) (layer "B.Cu") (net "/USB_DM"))
 (segment (start 44.96 41.79) (end 45.95 40.8) (width 0.22) (layer "B.Cu") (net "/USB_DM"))
 (segment (start 52.4 36.3) (end 52.4 37.28) (width 0.22) (layer "F.Cu") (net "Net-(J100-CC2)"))
 (segment (start 45.5 39.68) (end 45.5 42.55) (width 0.2) (layer "F.Cu") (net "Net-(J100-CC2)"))
 (via (at 52.4 37.28) (size 0.6) (drill 0.3) (layers "F.Cu" "B.Cu") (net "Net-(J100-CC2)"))
 (via (at 45.5 42.55) (size 0.6) (drill 0.3) (layers "F.Cu" "B.Cu") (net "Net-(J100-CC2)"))
 (segment (start 45.5 42.55) (end 49.8 42.55) (width 0.22) (layer "B.Cu") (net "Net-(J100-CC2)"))
 (segment (start 49.8 42.55) (end 52.4 39.95) (width 0.22) (layer "B.Cu") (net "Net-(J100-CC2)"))
 (segment (start 52.4 39.95) (end 52.4 37.28) (width 0.22) (layer "B.Cu") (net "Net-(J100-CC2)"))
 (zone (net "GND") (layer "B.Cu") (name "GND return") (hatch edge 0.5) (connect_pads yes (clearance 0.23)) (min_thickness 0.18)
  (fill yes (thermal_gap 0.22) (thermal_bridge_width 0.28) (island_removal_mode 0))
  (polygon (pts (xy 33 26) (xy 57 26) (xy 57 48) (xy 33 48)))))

